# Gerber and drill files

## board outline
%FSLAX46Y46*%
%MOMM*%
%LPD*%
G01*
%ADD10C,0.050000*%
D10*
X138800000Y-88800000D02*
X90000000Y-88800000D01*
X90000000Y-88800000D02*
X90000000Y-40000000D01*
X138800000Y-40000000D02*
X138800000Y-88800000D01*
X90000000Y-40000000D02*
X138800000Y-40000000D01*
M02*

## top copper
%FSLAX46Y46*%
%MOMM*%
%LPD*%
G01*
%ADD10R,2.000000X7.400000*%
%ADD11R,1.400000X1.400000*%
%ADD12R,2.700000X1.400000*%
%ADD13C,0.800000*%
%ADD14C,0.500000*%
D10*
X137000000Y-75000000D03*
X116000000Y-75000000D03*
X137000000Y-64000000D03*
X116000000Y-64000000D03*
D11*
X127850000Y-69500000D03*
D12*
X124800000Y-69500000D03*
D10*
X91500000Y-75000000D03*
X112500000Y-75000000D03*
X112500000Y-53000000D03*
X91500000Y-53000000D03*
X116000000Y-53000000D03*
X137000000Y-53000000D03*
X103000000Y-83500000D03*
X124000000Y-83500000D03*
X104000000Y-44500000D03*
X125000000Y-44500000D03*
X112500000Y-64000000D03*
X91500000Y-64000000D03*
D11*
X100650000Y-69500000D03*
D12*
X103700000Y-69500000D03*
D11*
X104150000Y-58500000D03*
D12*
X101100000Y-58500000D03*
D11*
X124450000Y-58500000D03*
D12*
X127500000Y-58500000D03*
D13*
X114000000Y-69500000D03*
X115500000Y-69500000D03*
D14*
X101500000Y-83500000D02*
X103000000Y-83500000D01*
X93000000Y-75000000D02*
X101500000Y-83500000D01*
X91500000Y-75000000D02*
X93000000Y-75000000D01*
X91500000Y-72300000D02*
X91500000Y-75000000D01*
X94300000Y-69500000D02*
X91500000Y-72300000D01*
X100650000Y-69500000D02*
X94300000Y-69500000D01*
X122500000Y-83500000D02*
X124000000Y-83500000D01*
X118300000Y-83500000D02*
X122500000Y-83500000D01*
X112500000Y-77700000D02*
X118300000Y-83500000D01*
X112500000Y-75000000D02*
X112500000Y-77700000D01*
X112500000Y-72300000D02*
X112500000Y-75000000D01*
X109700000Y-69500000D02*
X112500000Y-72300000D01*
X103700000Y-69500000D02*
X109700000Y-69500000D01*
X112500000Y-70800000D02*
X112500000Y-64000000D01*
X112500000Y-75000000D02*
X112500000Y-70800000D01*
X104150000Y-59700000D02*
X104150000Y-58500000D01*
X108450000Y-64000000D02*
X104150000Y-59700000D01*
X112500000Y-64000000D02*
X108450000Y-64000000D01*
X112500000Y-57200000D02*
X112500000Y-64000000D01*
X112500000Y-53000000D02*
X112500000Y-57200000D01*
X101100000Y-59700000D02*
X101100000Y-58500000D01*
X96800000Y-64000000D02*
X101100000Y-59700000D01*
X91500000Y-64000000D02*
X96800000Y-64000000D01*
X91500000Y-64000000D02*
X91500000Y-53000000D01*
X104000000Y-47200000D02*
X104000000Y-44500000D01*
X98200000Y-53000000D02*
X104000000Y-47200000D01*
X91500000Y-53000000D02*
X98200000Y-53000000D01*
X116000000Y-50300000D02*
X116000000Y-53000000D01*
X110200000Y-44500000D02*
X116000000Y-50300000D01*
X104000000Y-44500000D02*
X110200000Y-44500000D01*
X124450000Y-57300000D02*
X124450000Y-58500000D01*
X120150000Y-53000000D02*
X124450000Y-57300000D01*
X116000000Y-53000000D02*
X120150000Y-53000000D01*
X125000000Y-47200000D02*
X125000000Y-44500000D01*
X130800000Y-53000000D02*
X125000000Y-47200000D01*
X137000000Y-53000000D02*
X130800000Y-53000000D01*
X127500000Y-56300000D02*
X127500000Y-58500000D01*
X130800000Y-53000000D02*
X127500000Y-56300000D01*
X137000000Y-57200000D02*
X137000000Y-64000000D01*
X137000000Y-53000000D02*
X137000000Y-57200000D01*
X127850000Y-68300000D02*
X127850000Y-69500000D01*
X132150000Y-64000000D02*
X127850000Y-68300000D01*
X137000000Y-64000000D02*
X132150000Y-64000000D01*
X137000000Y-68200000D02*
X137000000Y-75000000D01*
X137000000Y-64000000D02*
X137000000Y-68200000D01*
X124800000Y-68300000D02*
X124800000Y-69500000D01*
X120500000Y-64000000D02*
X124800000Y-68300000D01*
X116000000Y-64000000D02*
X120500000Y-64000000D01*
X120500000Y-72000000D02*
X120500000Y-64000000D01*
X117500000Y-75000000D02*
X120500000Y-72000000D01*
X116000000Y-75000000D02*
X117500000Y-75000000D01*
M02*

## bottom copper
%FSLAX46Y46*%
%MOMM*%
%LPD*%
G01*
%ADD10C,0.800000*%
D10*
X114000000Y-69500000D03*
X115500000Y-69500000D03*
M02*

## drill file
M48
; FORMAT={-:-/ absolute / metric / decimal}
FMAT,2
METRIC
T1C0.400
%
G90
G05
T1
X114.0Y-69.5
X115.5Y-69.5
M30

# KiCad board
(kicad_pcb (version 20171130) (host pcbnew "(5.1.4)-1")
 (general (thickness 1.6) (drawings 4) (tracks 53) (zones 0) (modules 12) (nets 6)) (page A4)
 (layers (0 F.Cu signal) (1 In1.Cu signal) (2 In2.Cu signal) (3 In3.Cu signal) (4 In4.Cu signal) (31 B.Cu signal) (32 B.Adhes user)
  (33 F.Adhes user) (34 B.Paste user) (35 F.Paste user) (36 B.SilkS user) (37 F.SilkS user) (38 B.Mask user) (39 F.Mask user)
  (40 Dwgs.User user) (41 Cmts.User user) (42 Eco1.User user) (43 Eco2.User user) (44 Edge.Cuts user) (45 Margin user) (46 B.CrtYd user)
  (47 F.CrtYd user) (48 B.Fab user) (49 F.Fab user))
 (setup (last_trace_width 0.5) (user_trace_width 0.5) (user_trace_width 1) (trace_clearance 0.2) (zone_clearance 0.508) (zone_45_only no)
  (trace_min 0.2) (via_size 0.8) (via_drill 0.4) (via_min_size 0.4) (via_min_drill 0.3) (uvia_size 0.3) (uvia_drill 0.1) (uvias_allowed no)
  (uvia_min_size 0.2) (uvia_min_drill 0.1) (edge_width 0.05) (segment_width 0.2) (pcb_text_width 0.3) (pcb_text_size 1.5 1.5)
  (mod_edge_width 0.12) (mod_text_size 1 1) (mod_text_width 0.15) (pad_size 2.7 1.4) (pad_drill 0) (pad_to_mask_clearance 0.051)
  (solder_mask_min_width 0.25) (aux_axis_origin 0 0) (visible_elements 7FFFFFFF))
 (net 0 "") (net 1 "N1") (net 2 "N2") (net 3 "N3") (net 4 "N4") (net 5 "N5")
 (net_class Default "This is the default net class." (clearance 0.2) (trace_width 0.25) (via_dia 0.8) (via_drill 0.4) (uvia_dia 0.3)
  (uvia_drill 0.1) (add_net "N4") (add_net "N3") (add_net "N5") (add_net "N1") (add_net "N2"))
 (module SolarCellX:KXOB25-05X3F (layer F.Cu) (at 116 75)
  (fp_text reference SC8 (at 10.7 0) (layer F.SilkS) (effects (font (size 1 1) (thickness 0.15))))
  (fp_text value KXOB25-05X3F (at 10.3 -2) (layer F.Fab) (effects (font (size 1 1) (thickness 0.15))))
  (pad 2 smd rect (at 21 0) (size 2 7.4) (layers F.Cu F.Paste F.Mask) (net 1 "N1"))
  (pad 1 smd rect (at 0 0) (size 2 7.4) (layers F.Cu F.Paste F.Mask) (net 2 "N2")))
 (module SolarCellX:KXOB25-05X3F (layer F.Cu) (at 116 64)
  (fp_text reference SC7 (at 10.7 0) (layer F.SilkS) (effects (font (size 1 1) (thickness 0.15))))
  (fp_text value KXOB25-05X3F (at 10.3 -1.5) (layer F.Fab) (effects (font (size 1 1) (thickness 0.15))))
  (pad 2 smd rect (at 21 0) (size 2 7.4) (layers F.Cu F.Paste F.Mask) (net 1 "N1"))
  (pad 1 smd rect (at 0 0) (size 2 7.4) (layers F.Cu F.Paste F.Mask) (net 2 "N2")))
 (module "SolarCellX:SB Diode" (layer F.Cu) (at 126 69.5)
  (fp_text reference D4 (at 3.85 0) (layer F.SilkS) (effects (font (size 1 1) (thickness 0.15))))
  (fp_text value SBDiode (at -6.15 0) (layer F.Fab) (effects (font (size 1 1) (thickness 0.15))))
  (pad 2 smd rect (at 1.85 0) (size 1.4 1.4) (layers F.Cu F.Paste F.Mask) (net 1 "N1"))
  (pad 1 smd rect (at -1.2 0) (size 2.7 1.4) (layers F.Cu F.Paste F.Mask) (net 2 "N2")))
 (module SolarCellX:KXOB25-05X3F (layer F.Cu) (at 112.5 75 180)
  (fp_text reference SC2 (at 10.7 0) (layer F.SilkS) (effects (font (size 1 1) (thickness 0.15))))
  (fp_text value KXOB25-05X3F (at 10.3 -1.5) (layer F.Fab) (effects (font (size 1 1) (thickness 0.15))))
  (pad 2 smd rect (at 21 0 180) (size 2 7.4) (layers F.Cu F.Paste F.Mask) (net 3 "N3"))
  (pad 1 smd rect (at 0 0 180) (size 2 7.4) (layers F.Cu F.Paste F.Mask) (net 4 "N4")))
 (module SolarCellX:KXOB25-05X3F (layer F.Cu) (at 91.5 53)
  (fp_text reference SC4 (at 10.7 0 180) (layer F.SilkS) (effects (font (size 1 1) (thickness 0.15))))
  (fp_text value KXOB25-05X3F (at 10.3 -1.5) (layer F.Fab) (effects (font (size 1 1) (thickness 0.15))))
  (pad 2 smd rect (at 21 0) (size 2 7.4) (layers F.Cu F.Paste F.Mask) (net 4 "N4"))
  (pad 1 smd rect (at 0 0) (size 2 7.4) (layers F.Cu F.Paste F.Mask) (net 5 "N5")))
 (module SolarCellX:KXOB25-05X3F (layer F.Cu) (at 137 53 180)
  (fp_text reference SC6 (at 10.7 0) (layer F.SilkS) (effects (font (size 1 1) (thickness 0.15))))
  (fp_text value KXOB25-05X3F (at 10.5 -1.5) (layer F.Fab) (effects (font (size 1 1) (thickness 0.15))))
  (pad 2 smd rect (at 21 0 180) (size 2 7.4) (layers F.Cu F.Paste F.Mask) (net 5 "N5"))
  (pad 1 smd rect (at 0 0 180) (size 2 7.4) (layers F.Cu F.Paste F.Mask) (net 1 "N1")))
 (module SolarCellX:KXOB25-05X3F (layer F.Cu) (at 124 83.5 180)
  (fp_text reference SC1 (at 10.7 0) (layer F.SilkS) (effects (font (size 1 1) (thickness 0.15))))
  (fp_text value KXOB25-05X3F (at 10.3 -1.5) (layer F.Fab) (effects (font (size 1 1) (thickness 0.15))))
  (pad 2 smd rect (at 21 0 180) (size 2 7.4) (layers F.Cu F.Paste F.Mask) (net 3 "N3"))
  (pad 1 smd rect (at 0 0 180) (size 2 7.4) (layers F.Cu F.Paste F.Mask) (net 4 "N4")))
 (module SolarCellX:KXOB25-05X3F (layer F.Cu) (at 125 44.5 180)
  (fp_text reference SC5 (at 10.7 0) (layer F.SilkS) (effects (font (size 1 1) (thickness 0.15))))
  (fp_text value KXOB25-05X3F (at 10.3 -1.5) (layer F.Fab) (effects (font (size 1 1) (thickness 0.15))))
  (pad 2 smd rect (at 21 0 180) (size 2 7.4) (layers F.Cu F.Paste F.Mask) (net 5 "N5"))
  (pad 1 smd rect (at 0 0 180) (size 2 7.4) (layers F.Cu F.Paste F.Mask) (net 1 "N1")))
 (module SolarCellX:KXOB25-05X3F (layer F.Cu) (at 91.5 64)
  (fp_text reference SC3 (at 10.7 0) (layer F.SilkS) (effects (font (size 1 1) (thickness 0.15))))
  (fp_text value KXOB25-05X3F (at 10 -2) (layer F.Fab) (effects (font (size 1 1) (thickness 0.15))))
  (pad 2 smd rect (at 21 0) (size 2 7.4) (layers F.Cu F.Paste F.Mask) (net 4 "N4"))
  (pad 1 smd rect (at 0 0) (size 2 7.4) (layers F.Cu F.Paste F.Mask) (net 5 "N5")))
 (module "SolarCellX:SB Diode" (layer F.Cu) (at 102.5 69.5 180)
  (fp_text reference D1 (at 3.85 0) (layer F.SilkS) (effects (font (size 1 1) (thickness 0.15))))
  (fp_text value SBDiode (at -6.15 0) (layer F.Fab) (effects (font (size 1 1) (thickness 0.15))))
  (pad 2 smd rect (at 1.85 0 180) (size 1.4 1.4) (layers F.Cu F.Paste F.Mask) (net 3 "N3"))
  (pad 1 smd rect (at -1.2 0 180) (size 2.7 1.4) (layers F.Cu F.Paste F.Mask) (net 4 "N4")))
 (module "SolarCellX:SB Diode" (layer F.Cu) (at 102.3 58.5)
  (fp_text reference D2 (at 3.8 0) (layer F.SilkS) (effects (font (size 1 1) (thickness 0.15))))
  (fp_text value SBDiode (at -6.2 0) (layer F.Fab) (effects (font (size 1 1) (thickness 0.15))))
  (pad 2 smd rect (at 1.85 0) (size 1.4 1.4) (layers F.Cu F.Paste F.Mask) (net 4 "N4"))
  (pad 1 smd rect (at -1.2 0) (size 2.7 1.4) (layers F.Cu F.Paste F.Mask) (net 5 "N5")))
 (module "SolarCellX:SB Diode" (layer F.Cu) (at 126.3 58.5 180)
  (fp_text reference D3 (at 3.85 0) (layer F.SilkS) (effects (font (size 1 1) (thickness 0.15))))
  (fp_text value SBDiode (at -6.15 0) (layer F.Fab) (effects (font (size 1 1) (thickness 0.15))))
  (pad 2 smd rect (at 1.85 0 180) (size 1.4 1.4) (layers F.Cu F.Paste F.Mask) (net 5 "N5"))
  (pad 1 smd rect (at -1.2 0 180) (size 2.7 1.4) (layers F.Cu F.Paste F.Mask) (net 1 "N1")))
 (gr_line (start 138.8 88.8) (end 90 88.8) (layer Edge.Cuts) (width 0.05))
 (gr_line (start 90 88.8) (end 90 40) (layer Edge.Cuts) (width 0.05))
 (gr_line (start 138.8 40) (end 138.8 88.8) (layer Edge.Cuts) (width 0.05))
 (gr_line (start 90 40) (end 138.8 40) (layer Edge.Cuts) (width 0.05))
 (via (at 114 69.5) (size 0.8) (drill 0.4) (layers F.Cu B.Cu) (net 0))
 (via (at 115.5 69.5) (size 0.8) (drill 0.4) (layers F.Cu B.Cu) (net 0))
 (segment (start 101.5 83.5) (end 103 83.5) (width 0.5) (layer F.Cu) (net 3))
 (segment (start 93 75) (end 101.5 83.5) (width 0.5) (layer F.Cu) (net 3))
 (segment (start 91.5 75) (end 93 75) (width 0.5) (layer F.Cu) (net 3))
 (segment (start 91.5 72.3) (end 91.5 75) (width 0.5) (layer F.Cu) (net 3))
 (segment (start 94.3 69.5) (end 91.5 72.3) (width 0.5) (layer F.Cu) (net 3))
 (segment (start 100.65 69.5) (end 94.3 69.5) (width 0.5) (layer F.Cu) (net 3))
 (segment (start 122.5 83.5) (end 124 83.5) (width 0.5) (layer F.Cu) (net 4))
 (segment (start 118.3 83.5) (end 122.5 83.5) (width 0.5) (layer F.Cu) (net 4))
 (segment (start 112.5 77.7) (end 118.3 83.5) (width 0.5) (layer F.Cu) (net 4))
 (segment (start 112.5 75) (end 112.5 77.7) (width 0.5) (layer F.Cu) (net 4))
 (segment (start 112.5 72.3) (end 112.5 75) (width 0.5) (layer F.Cu) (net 4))
 (segment (start 109.7 69.5) (end 112.5 72.3) (width 0.5) (layer F.Cu) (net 4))
 (segment (start 103.7 69.5) (end 109.7 69.5) (width 0.5) (layer F.Cu) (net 4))
 (segment (start 112.5 70.8) (end 112.5 64) (width 0.5) (layer F.Cu) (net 4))
 (segment (start 112.5 75) (end 112.5 70.8) (width 0.5) (layer F.Cu) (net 4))
 (segment (start 104.15 59.7) (end 104.15 58.5) (width 0.5) (layer F.Cu) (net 4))
 (segment (start 108.45 64) (end 104.15 59.7) (width 0.5) (layer F.Cu) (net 4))
 (segment (start 112.5 64) (end 108.45 64) (width 0.5) (layer F.Cu) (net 4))
 (segment (start 112.5 57.2) (end 112.5 64) (width 0.5) (layer F.Cu) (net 4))
 (segment (start 112.5 53) (end 112.5 57.2) (width 0.5) (layer F.Cu) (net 4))
 (segment (start 101.1 59.7) (end 101.1 58.5) (width 0.5) (layer F.Cu) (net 5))
 (segment (start 96.8 64) (end 101.1 59.7) (width 0.5) (layer F.Cu) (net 5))
 (segment (start 91.5 64) (end 96.8 64) (width 0.5) (layer F.Cu) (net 5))
 (segment (start 91.5 64) (end 91.5 53) (width 0.5) (layer F.Cu) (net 5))
 (segment (start 104 47.2) (end 104 44.5) (width 0.5) (layer F.Cu) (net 5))
 (segment (start 98.2 53) (end 104 47.2) (width 0.5) (layer F.Cu) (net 5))
 (segment (start 91.5 53) (end 98.2 53) (width 0.5) (layer F.Cu) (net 5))
 (segment (start 116 50.3) (end 116 53) (width 0.5) (layer F.Cu) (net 5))
 (segment (start 110.2 44.5) (end 116 50.3) (width 0.5) (layer F.Cu) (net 5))
 (segment (start 104 44.5) (end 110.2 44.5) (width 0.5) (layer F.Cu) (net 5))
 (segment (start 124.45 57.3) (end 124.45 58.5) (width 0.5) (layer F.Cu) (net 5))
 (segment (start 120.15 53) (end 124.45 57.3) (width 0.5) (layer F.Cu) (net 5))
 (segment (start 116 53) (end 120.15 53) (width 0.5) (layer F.Cu) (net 5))
 (segment (start 125 47.2) (end 125 44.5) (width 0.5) (layer F.Cu) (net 1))
 (segment (start 130.8 53) (end 125 47.2) (width 0.5) (layer F.Cu) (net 1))
 (segment (start 137 53) (end 130.8 53) (width 0.5) (layer F.Cu) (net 1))
 (segment (start 127.5 56.3) (end 127.5 58.5) (width 0.5) (layer F.Cu) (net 1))
 (segment (start 130.8 53) (end 127.5 56.3) (width 0.5) (layer F.Cu) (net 1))
 (segment (start 137 57.2) (end 137 64) (width 0.5) (layer F.Cu) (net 1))
 (segment (start 137 53) (end 137 57.2) (width 0.5) (layer F.Cu) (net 1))
 (segment (start 127.85 68.3) (end 127.85 69.5) (width 0.5) (layer F.Cu) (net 1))
 (segment (start 132.15 64) (end 127.85 68.3) (width 0.5) (layer F.Cu) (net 1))
 (segment (start 137 64) (end 132.15 64) (width 0.5) (layer F.Cu) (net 1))
 (segment (start 137 68.2) (end 137 75) (width 0.5) (layer F.Cu) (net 1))
 (segment (start 137 64) (end 137 68.2) (width 0.5) (layer F.Cu) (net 1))
 (segment (start 124.8 68.3) (end 124.8 69.5) (width 0.5) (layer F.Cu) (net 2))
 (segment (start 120.5 64) (end 124.8 68.3) (width 0.5) (layer F.Cu) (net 2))
 (segment (start 116 64) (end 120.5 64) (width 0.5) (layer F.Cu) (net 2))
 (segment (start 120.5 72) (end 120.5 64) (width 0.5) (layer F.Cu) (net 2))
 (segment (start 117.5 75) (end 120.5 72) (width 0.5) (layer F.Cu) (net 2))
 (segment (start 116 75) (end 117.5 75) (width 0.5) (layer F.Cu) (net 2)))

